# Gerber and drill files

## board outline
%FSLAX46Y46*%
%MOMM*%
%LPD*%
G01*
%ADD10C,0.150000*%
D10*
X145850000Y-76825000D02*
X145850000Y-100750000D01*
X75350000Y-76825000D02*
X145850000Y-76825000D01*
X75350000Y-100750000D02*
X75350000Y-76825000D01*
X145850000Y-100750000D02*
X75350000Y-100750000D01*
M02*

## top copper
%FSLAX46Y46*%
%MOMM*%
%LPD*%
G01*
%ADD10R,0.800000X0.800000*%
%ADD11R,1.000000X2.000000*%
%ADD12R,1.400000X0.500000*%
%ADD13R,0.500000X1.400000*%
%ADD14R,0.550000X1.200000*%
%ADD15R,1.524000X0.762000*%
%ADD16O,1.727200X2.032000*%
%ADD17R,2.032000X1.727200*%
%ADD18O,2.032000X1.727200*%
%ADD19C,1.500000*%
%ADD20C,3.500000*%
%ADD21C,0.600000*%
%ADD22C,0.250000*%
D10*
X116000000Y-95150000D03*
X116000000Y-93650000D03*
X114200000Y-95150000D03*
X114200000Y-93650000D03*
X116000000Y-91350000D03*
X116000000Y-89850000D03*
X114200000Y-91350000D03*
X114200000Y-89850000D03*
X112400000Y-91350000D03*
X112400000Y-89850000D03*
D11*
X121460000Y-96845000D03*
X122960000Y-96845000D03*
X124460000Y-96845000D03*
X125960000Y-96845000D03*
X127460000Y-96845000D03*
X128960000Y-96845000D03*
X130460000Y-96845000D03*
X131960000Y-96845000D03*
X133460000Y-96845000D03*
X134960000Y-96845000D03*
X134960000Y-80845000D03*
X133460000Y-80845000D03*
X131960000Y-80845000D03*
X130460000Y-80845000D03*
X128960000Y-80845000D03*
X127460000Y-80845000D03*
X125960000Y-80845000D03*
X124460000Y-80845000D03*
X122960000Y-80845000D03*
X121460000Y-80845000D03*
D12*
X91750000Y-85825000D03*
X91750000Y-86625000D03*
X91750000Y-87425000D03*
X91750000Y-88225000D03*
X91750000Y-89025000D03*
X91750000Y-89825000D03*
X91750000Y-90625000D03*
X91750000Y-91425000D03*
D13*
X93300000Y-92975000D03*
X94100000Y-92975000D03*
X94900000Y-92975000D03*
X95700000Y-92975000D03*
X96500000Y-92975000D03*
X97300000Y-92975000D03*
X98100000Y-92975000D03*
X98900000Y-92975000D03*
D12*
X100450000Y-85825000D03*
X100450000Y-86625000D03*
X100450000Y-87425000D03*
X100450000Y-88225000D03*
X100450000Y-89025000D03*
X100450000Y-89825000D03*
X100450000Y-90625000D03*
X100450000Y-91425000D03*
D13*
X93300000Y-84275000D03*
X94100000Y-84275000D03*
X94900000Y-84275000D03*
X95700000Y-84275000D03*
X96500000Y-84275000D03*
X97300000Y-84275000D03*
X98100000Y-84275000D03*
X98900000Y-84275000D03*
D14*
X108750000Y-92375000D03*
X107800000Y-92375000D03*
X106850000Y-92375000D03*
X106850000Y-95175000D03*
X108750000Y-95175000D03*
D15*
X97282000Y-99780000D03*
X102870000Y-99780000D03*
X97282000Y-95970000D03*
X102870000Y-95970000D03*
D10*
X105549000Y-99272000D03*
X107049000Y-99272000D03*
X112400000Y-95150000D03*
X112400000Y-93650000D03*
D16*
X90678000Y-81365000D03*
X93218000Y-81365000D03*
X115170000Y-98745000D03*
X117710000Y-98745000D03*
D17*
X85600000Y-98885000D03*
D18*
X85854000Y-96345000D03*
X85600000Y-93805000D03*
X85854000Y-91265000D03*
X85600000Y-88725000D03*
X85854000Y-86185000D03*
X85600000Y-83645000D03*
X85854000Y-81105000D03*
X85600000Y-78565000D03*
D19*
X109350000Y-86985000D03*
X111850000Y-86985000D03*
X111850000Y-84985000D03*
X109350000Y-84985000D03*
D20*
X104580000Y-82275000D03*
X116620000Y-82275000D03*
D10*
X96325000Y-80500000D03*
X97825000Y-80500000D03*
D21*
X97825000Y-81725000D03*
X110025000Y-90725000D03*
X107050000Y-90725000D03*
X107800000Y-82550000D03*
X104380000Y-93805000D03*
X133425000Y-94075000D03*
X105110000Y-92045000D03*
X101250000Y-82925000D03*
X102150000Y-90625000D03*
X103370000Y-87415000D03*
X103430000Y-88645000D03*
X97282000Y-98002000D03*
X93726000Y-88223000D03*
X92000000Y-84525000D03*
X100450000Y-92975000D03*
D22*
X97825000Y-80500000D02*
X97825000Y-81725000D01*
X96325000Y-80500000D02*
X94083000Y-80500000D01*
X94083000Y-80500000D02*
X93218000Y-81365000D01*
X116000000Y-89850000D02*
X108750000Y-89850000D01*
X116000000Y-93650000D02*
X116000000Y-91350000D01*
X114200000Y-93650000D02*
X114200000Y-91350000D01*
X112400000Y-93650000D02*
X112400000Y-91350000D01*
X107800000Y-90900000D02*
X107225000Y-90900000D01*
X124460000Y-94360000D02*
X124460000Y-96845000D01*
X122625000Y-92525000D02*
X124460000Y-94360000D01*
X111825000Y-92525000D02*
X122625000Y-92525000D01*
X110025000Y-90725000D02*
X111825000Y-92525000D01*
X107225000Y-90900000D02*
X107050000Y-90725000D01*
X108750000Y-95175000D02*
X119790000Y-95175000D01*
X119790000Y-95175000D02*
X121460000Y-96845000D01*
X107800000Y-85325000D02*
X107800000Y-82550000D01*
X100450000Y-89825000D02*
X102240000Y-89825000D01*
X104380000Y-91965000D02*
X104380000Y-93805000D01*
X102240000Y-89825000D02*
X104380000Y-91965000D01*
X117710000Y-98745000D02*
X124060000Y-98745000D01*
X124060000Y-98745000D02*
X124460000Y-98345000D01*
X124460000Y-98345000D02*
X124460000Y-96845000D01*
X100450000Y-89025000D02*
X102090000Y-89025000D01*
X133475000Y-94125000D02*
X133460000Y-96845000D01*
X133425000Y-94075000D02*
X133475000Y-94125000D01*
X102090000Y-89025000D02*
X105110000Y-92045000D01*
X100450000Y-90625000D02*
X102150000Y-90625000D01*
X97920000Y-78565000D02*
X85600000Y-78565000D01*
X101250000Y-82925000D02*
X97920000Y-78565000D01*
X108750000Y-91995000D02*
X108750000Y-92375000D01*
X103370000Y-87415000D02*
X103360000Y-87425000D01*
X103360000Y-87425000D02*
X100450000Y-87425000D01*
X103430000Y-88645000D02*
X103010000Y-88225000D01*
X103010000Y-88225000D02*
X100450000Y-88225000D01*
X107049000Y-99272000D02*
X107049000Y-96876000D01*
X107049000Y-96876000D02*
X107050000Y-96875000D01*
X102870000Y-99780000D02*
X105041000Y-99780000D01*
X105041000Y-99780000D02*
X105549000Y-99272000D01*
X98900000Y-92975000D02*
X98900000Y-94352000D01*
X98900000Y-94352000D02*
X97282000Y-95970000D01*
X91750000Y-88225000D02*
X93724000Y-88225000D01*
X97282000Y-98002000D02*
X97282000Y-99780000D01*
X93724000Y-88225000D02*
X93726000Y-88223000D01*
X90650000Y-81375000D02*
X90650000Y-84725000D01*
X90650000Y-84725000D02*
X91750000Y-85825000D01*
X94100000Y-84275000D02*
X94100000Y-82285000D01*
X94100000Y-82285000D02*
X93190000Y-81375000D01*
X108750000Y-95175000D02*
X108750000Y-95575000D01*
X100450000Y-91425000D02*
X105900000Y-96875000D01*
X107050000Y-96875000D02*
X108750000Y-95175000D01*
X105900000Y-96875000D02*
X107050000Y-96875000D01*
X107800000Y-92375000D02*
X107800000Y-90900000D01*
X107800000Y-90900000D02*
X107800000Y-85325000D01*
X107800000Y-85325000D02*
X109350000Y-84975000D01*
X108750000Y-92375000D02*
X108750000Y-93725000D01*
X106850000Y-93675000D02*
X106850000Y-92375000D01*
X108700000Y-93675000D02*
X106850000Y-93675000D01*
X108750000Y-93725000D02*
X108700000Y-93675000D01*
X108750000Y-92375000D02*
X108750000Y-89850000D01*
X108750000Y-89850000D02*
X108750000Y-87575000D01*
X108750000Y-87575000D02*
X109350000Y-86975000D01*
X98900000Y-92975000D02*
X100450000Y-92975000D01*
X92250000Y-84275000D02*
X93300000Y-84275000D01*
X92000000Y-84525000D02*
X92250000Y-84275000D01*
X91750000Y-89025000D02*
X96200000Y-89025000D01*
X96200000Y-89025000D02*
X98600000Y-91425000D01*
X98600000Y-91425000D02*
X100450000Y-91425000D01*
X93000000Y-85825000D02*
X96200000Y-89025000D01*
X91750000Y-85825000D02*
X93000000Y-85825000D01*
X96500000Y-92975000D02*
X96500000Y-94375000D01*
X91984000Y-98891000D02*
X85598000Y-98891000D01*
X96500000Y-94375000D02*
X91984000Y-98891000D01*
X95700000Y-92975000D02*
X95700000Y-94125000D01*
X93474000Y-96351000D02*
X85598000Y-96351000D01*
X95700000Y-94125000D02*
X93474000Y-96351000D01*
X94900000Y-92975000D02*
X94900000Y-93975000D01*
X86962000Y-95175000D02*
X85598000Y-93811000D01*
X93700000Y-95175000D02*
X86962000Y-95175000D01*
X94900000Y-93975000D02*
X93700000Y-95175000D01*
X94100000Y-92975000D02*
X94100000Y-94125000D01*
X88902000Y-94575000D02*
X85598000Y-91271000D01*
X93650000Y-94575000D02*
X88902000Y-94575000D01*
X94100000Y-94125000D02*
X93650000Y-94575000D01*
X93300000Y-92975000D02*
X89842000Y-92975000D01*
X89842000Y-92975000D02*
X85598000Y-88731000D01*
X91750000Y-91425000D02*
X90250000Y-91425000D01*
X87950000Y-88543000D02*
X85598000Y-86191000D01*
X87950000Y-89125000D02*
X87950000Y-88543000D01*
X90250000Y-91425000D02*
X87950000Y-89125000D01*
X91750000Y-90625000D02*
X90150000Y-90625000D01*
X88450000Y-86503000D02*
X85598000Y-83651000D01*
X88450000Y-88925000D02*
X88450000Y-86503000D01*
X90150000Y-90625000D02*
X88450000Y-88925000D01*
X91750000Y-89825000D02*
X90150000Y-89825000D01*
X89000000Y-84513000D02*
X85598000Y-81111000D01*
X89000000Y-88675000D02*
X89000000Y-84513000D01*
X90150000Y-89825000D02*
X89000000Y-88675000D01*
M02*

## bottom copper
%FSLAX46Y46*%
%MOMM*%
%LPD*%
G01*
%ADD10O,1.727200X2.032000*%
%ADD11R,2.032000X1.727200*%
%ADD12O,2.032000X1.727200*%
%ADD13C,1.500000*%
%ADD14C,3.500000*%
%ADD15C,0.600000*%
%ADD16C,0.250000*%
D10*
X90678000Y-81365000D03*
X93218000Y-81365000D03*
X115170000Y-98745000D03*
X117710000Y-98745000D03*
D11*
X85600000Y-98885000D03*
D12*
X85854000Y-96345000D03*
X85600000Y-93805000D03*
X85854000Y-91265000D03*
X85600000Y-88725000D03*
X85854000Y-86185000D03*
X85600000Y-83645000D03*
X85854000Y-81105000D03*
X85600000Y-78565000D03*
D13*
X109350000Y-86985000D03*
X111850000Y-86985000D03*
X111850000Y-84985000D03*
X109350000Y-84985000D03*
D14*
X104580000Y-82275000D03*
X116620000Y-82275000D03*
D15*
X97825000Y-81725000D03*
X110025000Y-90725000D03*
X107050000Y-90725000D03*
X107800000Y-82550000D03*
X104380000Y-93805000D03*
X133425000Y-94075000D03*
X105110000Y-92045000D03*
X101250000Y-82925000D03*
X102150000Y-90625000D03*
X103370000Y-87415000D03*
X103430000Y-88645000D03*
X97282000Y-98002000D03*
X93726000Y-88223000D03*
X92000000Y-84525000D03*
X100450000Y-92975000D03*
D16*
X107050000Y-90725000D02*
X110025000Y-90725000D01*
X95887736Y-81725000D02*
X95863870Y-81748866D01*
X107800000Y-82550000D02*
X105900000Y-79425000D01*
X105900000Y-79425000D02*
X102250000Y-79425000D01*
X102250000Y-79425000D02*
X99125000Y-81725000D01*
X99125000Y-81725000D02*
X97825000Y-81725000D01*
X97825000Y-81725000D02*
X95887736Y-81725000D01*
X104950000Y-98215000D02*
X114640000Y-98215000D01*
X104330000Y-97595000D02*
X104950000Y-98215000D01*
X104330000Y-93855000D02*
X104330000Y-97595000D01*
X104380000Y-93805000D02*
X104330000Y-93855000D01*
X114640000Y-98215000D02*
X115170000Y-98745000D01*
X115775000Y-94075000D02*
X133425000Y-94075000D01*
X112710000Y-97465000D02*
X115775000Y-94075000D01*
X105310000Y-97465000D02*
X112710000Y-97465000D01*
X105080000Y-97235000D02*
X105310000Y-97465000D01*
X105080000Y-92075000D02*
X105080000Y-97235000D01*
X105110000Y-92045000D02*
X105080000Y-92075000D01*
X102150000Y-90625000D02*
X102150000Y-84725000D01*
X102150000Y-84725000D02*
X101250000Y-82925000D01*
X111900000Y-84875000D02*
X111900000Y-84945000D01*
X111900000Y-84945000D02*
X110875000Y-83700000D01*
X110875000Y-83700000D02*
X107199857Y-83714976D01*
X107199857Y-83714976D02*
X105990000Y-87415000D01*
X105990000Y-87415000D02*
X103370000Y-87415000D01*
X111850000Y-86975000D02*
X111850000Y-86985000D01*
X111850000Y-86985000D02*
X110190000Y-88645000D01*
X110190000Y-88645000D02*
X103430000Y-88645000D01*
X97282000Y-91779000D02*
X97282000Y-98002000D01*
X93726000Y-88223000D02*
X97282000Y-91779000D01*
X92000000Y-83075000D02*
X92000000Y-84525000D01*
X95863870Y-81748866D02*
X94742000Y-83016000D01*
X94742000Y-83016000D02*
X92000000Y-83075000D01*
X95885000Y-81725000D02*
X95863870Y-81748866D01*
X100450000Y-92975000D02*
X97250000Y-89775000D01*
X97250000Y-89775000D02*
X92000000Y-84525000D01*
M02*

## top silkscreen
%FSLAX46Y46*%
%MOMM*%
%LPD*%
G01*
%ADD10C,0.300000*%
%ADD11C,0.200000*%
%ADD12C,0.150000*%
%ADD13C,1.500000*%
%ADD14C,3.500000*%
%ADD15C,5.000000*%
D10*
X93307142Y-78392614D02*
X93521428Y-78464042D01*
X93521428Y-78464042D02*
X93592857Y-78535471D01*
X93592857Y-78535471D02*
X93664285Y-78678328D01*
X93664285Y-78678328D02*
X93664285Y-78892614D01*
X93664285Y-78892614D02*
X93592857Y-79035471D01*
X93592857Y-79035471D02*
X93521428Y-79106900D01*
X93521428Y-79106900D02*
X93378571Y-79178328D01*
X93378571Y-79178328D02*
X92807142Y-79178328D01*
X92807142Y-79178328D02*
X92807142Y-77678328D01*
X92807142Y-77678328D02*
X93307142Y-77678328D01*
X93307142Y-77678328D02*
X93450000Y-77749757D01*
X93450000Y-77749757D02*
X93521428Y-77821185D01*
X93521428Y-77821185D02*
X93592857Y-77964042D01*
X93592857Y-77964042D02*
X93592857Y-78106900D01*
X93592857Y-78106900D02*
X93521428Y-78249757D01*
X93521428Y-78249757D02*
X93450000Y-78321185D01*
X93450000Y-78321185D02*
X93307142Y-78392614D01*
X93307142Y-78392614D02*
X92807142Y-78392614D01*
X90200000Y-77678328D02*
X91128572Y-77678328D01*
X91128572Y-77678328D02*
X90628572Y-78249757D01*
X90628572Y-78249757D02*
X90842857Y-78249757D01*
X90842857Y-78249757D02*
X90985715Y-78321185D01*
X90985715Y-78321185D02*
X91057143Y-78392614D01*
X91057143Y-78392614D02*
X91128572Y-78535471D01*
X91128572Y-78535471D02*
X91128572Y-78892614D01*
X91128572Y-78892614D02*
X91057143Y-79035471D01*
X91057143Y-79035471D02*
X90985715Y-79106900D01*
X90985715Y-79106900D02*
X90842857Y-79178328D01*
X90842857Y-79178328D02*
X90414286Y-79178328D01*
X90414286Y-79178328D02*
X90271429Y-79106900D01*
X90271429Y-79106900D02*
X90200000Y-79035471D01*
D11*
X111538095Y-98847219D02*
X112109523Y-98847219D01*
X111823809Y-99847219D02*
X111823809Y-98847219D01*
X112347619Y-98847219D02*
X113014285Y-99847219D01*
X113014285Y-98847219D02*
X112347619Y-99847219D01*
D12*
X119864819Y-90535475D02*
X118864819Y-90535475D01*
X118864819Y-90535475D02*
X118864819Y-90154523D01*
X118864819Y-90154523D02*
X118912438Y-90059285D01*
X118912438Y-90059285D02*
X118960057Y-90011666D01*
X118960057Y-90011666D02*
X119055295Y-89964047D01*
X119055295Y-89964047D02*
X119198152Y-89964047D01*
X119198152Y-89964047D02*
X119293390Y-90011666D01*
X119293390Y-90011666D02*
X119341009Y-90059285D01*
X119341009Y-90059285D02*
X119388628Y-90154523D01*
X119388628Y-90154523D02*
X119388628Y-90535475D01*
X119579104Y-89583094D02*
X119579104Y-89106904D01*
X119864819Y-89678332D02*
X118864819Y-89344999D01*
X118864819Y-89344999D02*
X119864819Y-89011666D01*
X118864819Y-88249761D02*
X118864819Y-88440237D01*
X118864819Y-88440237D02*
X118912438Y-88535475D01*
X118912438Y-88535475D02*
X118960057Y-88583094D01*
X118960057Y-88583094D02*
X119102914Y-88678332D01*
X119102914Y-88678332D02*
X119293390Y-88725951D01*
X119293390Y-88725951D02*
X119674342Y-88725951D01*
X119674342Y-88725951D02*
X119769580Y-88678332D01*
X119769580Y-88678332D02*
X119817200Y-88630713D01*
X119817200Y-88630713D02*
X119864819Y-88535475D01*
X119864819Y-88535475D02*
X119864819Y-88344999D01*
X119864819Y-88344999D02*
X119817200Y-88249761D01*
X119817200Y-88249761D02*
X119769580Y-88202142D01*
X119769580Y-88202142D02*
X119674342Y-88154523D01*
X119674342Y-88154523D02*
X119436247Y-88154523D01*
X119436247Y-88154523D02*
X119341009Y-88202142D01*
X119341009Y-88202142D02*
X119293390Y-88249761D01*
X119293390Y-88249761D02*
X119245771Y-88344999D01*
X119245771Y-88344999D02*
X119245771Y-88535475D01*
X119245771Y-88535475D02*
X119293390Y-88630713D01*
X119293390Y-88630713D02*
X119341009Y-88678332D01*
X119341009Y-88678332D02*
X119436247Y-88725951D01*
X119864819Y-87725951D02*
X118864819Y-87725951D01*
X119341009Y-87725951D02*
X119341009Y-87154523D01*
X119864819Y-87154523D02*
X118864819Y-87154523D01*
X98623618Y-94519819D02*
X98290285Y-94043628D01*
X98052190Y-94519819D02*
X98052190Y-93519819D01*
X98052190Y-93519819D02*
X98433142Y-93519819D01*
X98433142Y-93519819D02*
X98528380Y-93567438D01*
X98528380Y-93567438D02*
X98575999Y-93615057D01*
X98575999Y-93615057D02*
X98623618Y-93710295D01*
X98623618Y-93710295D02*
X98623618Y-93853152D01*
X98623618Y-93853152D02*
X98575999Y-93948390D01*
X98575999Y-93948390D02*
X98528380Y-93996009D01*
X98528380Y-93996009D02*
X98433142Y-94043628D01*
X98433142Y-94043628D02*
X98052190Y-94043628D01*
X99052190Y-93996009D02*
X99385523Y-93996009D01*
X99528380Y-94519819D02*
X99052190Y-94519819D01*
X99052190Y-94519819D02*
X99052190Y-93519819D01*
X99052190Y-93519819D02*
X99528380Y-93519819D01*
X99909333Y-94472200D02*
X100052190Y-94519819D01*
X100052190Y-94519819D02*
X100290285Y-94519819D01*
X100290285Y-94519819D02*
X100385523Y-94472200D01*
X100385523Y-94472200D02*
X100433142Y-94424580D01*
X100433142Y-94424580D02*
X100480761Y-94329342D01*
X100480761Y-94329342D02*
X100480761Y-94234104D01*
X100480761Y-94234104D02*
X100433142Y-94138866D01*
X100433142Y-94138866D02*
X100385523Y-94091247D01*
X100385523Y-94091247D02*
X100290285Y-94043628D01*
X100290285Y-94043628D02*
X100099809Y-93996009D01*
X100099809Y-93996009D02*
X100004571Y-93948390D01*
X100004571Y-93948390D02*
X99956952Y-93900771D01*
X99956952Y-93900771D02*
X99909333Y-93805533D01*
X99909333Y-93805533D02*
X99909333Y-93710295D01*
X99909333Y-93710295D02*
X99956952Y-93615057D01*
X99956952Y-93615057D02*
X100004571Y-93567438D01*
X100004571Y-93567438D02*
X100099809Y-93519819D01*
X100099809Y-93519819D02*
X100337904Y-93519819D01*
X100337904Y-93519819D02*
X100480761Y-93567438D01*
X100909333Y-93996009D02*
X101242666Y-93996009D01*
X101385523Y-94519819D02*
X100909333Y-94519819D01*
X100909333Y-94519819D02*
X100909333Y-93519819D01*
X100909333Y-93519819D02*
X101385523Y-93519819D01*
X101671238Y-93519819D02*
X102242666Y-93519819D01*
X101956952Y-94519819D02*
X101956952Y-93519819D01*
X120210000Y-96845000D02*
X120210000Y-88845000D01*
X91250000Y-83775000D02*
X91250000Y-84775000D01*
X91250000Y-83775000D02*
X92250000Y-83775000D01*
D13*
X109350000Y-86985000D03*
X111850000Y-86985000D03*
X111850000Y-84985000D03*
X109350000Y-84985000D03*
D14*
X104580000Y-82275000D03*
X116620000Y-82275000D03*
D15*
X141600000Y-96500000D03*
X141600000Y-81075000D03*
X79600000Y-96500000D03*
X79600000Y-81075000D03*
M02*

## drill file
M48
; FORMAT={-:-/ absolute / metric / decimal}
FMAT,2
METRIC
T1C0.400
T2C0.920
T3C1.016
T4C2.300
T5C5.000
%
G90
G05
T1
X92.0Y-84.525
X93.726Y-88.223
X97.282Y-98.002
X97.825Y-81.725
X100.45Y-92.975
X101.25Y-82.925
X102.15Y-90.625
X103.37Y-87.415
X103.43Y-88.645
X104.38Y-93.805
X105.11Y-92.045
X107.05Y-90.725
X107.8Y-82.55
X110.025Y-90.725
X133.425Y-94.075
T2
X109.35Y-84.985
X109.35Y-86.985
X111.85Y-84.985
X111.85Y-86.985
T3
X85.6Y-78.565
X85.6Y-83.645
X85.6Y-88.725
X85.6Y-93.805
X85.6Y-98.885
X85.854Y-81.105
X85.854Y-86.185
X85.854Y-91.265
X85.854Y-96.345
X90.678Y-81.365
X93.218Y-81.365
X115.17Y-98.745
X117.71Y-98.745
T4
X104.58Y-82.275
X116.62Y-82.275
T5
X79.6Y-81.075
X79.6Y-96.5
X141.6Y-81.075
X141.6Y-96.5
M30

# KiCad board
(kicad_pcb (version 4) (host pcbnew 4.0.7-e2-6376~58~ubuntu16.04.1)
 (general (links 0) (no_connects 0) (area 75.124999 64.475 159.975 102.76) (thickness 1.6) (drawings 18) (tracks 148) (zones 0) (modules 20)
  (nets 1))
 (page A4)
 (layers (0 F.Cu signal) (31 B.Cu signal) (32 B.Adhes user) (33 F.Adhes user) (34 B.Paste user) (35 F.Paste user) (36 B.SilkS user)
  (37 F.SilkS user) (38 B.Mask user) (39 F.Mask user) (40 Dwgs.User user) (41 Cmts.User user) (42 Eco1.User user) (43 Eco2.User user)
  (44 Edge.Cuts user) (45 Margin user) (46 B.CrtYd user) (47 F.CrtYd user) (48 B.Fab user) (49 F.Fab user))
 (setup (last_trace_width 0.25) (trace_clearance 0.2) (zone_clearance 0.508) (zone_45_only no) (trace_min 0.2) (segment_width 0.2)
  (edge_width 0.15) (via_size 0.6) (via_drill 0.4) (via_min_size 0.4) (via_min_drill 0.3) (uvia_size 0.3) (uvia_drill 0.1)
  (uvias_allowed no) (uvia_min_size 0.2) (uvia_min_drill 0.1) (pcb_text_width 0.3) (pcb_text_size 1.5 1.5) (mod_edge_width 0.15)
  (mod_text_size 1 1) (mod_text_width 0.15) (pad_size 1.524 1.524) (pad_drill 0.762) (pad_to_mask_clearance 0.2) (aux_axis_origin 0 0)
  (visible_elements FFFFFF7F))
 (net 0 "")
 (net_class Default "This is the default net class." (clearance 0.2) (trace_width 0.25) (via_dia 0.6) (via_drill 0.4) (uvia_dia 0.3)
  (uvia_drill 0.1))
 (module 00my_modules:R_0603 (layer F.Cu) (at 116 94.4 90)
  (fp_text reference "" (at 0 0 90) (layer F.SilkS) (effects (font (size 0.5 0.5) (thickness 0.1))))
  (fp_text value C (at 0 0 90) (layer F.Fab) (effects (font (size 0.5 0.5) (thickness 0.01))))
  (pad 1 smd rect (at -0.75 0 90) (size 0.8 0.8) (layers F.Cu F.Paste F.Mask))
  (pad 2 smd rect (at 0.75 0 90) (size 0.8 0.8) (layers F.Cu F.Paste F.Mask)))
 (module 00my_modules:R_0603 (layer F.Cu) (at 114.2 94.4 90)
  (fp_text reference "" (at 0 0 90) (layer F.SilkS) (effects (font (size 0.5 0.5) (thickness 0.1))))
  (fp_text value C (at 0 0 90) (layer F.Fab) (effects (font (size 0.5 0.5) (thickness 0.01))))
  (pad 1 smd rect (at -0.75 0 90) (size 0.8 0.8) (layers F.Cu F.Paste F.Mask))
  (pad 2 smd rect (at 0.75 0 90) (size 0.8 0.8) (layers F.Cu F.Paste F.Mask)))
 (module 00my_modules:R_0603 (layer F.Cu) (at 116 90.6 90)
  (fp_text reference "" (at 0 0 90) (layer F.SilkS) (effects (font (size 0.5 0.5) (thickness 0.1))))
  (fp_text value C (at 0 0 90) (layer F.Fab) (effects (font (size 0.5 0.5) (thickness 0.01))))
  (pad 1 smd rect (at -0.75 0 90) (size 0.8 0.8) (layers F.Cu F.Paste F.Mask))
  (pad 2 smd rect (at 0.75 0 90) (size 0.8 0.8) (layers F.Cu F.Paste F.Mask)))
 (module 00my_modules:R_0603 (layer F.Cu) (at 114.2 90.6 90)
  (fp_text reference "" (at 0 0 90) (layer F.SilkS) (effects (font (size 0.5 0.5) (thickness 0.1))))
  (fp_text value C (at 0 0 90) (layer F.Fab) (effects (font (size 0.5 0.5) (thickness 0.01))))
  (pad 1 smd rect (at -0.75 0 90) (size 0.8 0.8) (layers F.Cu F.Paste F.Mask))
  (pad 2 smd rect (at 0.75 0 90) (size 0.8 0.8) (layers F.Cu F.Paste F.Mask)))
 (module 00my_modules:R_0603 (layer F.Cu) (at 112.4 90.6 90)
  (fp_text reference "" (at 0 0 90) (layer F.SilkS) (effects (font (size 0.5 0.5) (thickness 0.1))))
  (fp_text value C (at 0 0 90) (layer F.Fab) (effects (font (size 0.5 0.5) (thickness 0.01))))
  (pad 1 smd rect (at -0.75 0 90) (size 0.8 0.8) (layers F.Cu F.Paste F.Mask))
  (pad 2 smd rect (at 0.75 0 90) (size 0.8 0.8) (layers F.Cu F.Paste F.Mask)))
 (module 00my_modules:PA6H (layer F.Cu) (at 128.21 88.845 90)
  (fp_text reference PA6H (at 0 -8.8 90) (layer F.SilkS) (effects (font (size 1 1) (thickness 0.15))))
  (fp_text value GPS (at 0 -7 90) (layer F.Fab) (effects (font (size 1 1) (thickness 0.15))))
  (fp_line (start -8 -8) (end 0 -8) (layer F.SilkS) (width 0.15))
  (pad VCC smd rect (at -8 -6.75 90) (size 2 1) (layers F.Cu F.Paste F.Mask))
  (pad 2 smd rect (at -8 -5.25 90) (size 2 1) (layers F.Cu F.Paste F.Mask))
  (pad GND smd rect (at -8 -3.75 90) (size 2 1) (layers F.Cu F.Paste F.Mask))
  (pad 4 smd rect (at -8 -2.25 90) (size 2 1) (layers F.Cu F.Paste F.Mask))
  (pad 5 smd rect (at -8 -0.75 90) (size 2 1) (layers F.Cu F.Paste F.Mask))
  (pad 6 smd rect (at -8 0.75 90) (size 2 1) (layers F.Cu F.Paste F.Mask))
  (pad 7 smd rect (at -8 2.25 90) (size 2 1) (layers F.Cu F.Paste F.Mask))
  (pad 8 smd rect (at -8 3.75 90) (size 2 1) (layers F.Cu F.Paste F.Mask))
  (pad TX smd rect (at -8 5.25 90) (size 2 1) (layers F.Cu F.Paste F.Mask))
  (pad RX smd rect (at -8 6.75 90) (size 2 1) (layers F.Cu F.Paste F.Mask))
  (pad 11 smd rect (at 8 6.75 90) (size 2 1) (layers F.Cu F.Paste F.Mask))
  (pad 12 smd rect (at 8 5.25 90) (size 2 1) (layers F.Cu F.Paste F.Mask))
  (pad 13 smd rect (at 8 3.75 90) (size 2 1) (layers F.Cu F.Paste F.Mask))
  (pad 14 smd rect (at 8 2.25 90) (size 2 1) (layers F.Cu F.Paste F.Mask))
  (pad 15 smd rect (at 8 0.75 90) (size 2 1) (layers F.Cu F.Paste F.Mask))
  (pad 16 smd rect (at 8 -0.75 90) (size 2 1) (layers F.Cu F.Paste F.Mask))
  (pad 17 smd rect (at 8 -2.25 90) (size 2 1) (layers F.Cu F.Paste F.Mask))
  (pad 18 smd rect (at 8 -3.75 90) (size 2 1) (layers F.Cu F.Paste F.Mask))
  (pad 19 smd rect (at 8 -5.25 90) (size 2 1) (layers F.Cu F.Paste F.Mask))
  (pad 20 smd rect (at 8 -6.75 90) (size 2 1) (layers F.Cu F.Paste F.Mask)))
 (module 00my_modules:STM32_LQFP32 (layer F.Cu) (at 96.1 88.625)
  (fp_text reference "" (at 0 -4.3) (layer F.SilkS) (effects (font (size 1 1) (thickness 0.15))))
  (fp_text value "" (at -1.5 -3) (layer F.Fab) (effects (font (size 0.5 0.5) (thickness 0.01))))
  (fp_line (start -4.85 -4.85) (end -4.85 -3.85) (layer F.SilkS) (width 0.15))
  (fp_line (start -4.85 -4.85) (end -3.85 -4.85) (layer F.SilkS) (width 0.15))
  (pad 3.3 smd rect (at -4.35 -2.8) (size 1.4 0.5) (layers F.Cu F.Paste F.Mask))
  (pad PF0 smd rect (at -4.35 -2) (size 1.4 0.5) (layers F.Cu F.Paste F.Mask))
  (pad PF1 smd rect (at -4.35 -1.2) (size 1.4 0.5) (layers F.Cu F.Paste F.Mask))
  (pad RST smd rect (at -4.35 -0.4) (size 1.4 0.5) (layers F.Cu F.Paste F.Mask))
  (pad 3.3 smd rect (at -4.35 0.4) (size 1.4 0.5) (layers F.Cu F.Paste F.Mask))
  (pad PA0 smd rect (at -4.35 1.2) (size 1.4 0.5) (layers F.Cu F.Paste F.Mask))
  (pad PA1 smd rect (at -4.35 2) (size 1.4 0.5) (layers F.Cu F.Paste F.Mask))
  (pad PA2 smd rect (at -4.35 2.8) (size 1.4 0.5) (layers F.Cu F.Paste F.Mask))
  (pad PA3 smd rect (at -2.8 4.35 90) (size 1.4 0.5) (layers F.Cu F.Paste F.Mask))
  (pad PA4 smd rect (at -2 4.35 90) (size 1.4 0.5) (layers F.Cu F.Paste F.Mask))
  (pad PA5 smd rect (at -1.2 4.35 90) (size 1.4 0.5) (layers F.Cu F.Paste F.Mask))
  (pad PA6 smd rect (at -0.4 4.35 90) (size 1.4 0.5) (layers F.Cu F.Paste F.Mask))
  (pad PA7 smd rect (at 0.4 4.35 90) (size 1.4 0.5) (layers F.Cu F.Paste F.Mask))
  (pad PB0 smd rect (at 1.2 4.35 90) (size 1.4 0.5) (layers F.Cu F.Paste F.Mask))
  (pad PB1 smd rect (at 2 4.35 90) (size 1.4 0.5) (layers F.Cu F.Paste F.Mask))
  (pad GND smd rect (at 2.8 4.35 90) (size 1.4 0.5) (layers F.Cu F.Paste F.Mask))
  (pad PA14 smd rect (at 4.35 -2.8) (size 1.4 0.5) (layers F.Cu F.Paste F.Mask))
  (pad PA13 smd rect (at 4.35 -2) (size 1.4 0.5) (layers F.Cu F.Paste F.Mask))
  (pad PA12 smd rect (at 4.35 -1.2) (size 1.4 0.5) (layers F.Cu F.Paste F.Mask))
  (pad PA11 smd rect (at 4.35 -0.4) (size 1.4 0.5) (layers F.Cu F.Paste F.Mask))
  (pad PA10 smd rect (at 4.35 0.4) (size 1.4 0.5) (layers F.Cu F.Paste F.Mask))
  (pad PA9 smd rect (at 4.35 1.2) (size 1.4 0.5) (layers F.Cu F.Paste F.Mask))
  (pad PA8 smd rect (at 4.35 2) (size 1.4 0.5) (layers F.Cu F.Paste F.Mask))
  (pad 3.3 smd rect (at 4.35 2.8) (size 1.4 0.5) (layers F.Cu F.Paste F.Mask))
  (pad GND smd rect (at -2.8 -4.35 90) (size 1.4 0.5) (layers F.Cu F.Paste F.Mask))
  (pad BOOT smd rect (at -2 -4.35 90) (size 1.4 0.5) (layers F.Cu F.Paste F.Mask))
  (pad PB7 smd rect (at -1.2 -4.35 90) (size 1.4 0.5) (layers F.Cu F.Paste F.Mask))
  (pad PB6 smd rect (at -0.4 -4.35 90) (size 1.4 0.5) (layers F.Cu F.Paste F.Mask))
  (pad PB5 smd rect (at 0.4 -4.35 90) (size 1.4 0.5) (layers F.Cu F.Paste F.Mask))
  (pad PB4 smd rect (at 1.2 -4.35 90) (size 1.4 0.5) (layers F.Cu F.Paste F.Mask))
  (pad PB3 smd rect (at 2 -4.35 90) (size 1.4 0.5) (layers F.Cu F.Paste F.Mask))
  (pad PA15 smd rect (at 2.8 -4.35 90) (size 1.4 0.5) (layers F.Cu F.Paste F.Mask)))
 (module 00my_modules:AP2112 (layer F.Cu) (at 107.8 93.775 270)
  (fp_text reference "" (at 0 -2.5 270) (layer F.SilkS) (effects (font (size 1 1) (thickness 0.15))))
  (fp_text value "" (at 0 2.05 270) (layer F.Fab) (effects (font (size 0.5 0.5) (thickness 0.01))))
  (pad VIN smd rect (at -1.4 -0.95 270) (size 1.2 0.55) (layers F.Cu F.Paste F.Mask))
  (pad GND smd rect (at -1.4 0 270) (size 1.2 0.55) (layers F.Cu F.Paste F.Mask))
  (pad EN smd rect (at -1.4 0.95 270) (size 1.2 0.55) (layers F.Cu F.Paste F.Mask))
  (pad NC smd rect (at 1.4 0.95 270) (size 1.2 0.55) (layers F.Cu F.Paste F.Mask))
  (pad VOUT smd rect (at 1.4 -0.95 270) (size 1.2 0.55) (layers F.Cu F.Paste F.Mask)))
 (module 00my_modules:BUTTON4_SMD (layer F.Cu) (at 100.076 97.875)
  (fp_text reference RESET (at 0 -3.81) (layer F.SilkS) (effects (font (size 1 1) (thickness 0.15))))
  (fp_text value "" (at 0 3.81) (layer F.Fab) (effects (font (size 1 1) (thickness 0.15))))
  (pad 1 smd rect (at -2.794 1.905) (size 1.524 0.762) (layers F.Cu F.Paste F.Mask))
  (pad 2 smd rect (at 2.794 1.905) (size 1.524 0.762) (layers F.Cu F.Paste F.Mask))
  (pad 3 smd rect (at -2.794 -1.905) (size 1.524 0.762) (layers F.Cu F.Paste F.Mask))
  (pad 4 smd rect (at 2.794 -1.905) (size 1.524 0.762) (layers F.Cu F.Paste F.Mask)))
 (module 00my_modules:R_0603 (layer F.Cu) (at 106.299 99.272)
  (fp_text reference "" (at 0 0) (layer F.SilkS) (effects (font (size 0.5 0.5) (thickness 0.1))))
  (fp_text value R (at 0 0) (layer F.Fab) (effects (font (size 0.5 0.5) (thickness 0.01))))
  (pad 1 smd rect (at -0.75 0) (size 0.8 0.8) (layers F.Cu F.Paste F.Mask))
  (pad 2 smd rect (at 0.75 0) (size 0.8 0.8) (layers F.Cu F.Paste F.Mask)))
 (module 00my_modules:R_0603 (layer F.Cu) (at 112.4 94.4 90)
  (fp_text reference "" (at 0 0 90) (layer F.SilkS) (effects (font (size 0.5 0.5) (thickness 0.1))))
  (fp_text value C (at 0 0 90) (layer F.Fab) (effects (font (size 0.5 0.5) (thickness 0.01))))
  (pad 1 smd rect (at -0.75 0 90) (size 0.8 0.8) (layers F.Cu F.Paste F.Mask))
  (pad 2 smd rect (at 0.75 0 90) (size 0.8 0.8) (layers F.Cu F.Paste F.Mask)))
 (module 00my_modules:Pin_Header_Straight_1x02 (layer B.Cu) (at 90.678 81.365 270)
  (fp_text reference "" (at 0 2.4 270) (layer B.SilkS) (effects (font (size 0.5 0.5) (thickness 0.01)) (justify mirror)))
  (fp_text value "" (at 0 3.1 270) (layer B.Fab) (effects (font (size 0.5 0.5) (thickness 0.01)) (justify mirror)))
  (pad 1 thru_hole oval (at 0 0 270) (size 2.032 1.7272) (drill 1.016) (layers *.Cu *.Mask B.SilkS))
  (pad 2 thru_hole oval (at 0 -2.54 270) (size 2.032 1.7272) (drill 1.016) (layers *.Cu *.Mask B.SilkS)))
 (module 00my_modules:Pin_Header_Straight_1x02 (layer B.Cu) (at 115.17 98.745 270)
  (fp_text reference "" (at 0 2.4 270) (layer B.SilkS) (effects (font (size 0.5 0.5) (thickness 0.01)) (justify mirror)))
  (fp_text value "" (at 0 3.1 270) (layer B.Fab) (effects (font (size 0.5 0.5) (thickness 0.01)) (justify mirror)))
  (pad 1 thru_hole oval (at 0 0 270) (size 2.032 1.7272) (drill 1.016) (layers *.Cu *.Mask B.SilkS))
  (pad 2 thru_hole oval (at 0 -2.54 270) (size 2.032 1.7272) (drill 1.016) (layers *.Cu *.Mask B.SilkS)))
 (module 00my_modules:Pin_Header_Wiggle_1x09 (layer B.Cu) (at 85.6 98.885)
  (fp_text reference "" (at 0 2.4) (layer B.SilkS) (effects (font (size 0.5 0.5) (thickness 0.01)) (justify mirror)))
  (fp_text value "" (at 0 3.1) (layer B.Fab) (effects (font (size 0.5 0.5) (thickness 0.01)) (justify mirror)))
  (pad 1 thru_hole rect (at 0 0) (size 2.032 1.7272) (drill 1.016) (layers *.Cu *.Mask B.SilkS))
  (pad 2 thru_hole oval (at 0.254 -2.54) (size 2.032 1.7272) (drill 1.016) (layers *.Cu *.Mask B.SilkS))
  (pad 3 thru_hole oval (at 0 -5.08) (size 2.032 1.7272) (drill 1.016) (layers *.Cu *.Mask B.SilkS))
  (pad 4 thru_hole oval (at 0.254 -7.62) (size 2.032 1.7272) (drill 1.016) (layers *.Cu *.Mask B.SilkS))
  (pad 5 thru_hole oval (at 0 -10.16) (size 2.032 1.7272) (drill 1.016) (layers *.Cu *.Mask B.SilkS))
  (pad 6 thru_hole oval (at 0.254 -12.7) (size 2.032 1.7272) (drill 1.016) (layers *.Cu *.Mask B.SilkS))
  (pad 7 thru_hole oval (at 0 -15.24) (size 2.032 1.7272) (drill 1.016) (layers *.Cu *.Mask B.SilkS))
  (pad 8 thru_hole oval (at 0.254 -17.78) (size 2.032 1.7272) (drill 1.016) (layers *.Cu *.Mask B.SilkS))
  (pad 9 thru_hole oval (at 0 -20.32) (size 2.032 1.7272) (drill 1.016) (layers *.Cu *.Mask B.SilkS)))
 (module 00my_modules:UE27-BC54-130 (layer F.Cu) (at 110.6 82.275 180)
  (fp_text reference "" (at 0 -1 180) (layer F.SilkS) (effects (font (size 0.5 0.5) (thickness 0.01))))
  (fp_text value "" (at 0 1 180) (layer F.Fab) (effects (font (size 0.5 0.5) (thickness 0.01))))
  (pad V thru_hole circle (at 1.25 -4.71 180) (size 1.5 1.5) (drill 0.92) (layers *.Cu *.Mask F.SilkS))
  (pad - thru_hole circle (at -1.25 -4.71 180) (size 1.5 1.5) (drill 0.92) (layers *.Cu *.Mask F.SilkS))
  (pad + thru_hole circle (at -1.25 -2.71 180) (size 1.5 1.5) (drill 0.92) (layers *.Cu *.Mask F.SilkS))
  (pad G thru_hole circle (at 1.25 -2.71 180) (size 1.5 1.5) (drill 0.92) (layers *.Cu *.Mask F.SilkS))
  (pad X thru_hole circle (at 6.02 0 180) (size 3.5 3.5) (drill 2.3) (layers *.Cu *.Mask F.SilkS))
  (pad X thru_hole circle (at -6.02 0 180) (size 3.5 3.5) (drill 2.3) (layers *.Cu *.Mask F.SilkS)))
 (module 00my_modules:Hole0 (layer F.Cu) (at 141.6 96.5)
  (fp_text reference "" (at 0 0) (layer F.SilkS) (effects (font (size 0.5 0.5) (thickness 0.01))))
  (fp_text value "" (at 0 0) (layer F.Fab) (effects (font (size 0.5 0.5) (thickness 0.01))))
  (pad "" np_thru_hole circle (at 0 0) (size 5 5) (drill 5) (layers *.Cu *.Mask F.SilkS)))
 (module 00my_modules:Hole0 (layer F.Cu) (at 141.6 81.075)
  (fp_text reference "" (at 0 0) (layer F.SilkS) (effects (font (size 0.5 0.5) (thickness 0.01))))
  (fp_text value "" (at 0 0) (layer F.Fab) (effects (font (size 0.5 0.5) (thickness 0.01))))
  (pad "" np_thru_hole circle (at 0 0) (size 5 5) (drill 5) (layers *.Cu *.Mask F.SilkS)))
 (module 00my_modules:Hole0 (layer F.Cu) (at 79.6 96.5)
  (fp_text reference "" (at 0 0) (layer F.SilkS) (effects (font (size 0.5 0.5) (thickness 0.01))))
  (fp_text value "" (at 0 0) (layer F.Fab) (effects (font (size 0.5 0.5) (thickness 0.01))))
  (pad "" np_thru_hole circle (at 0 0) (size 5 5) (drill 5) (layers *.Cu *.Mask F.SilkS)))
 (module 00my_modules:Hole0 (layer F.Cu) (at 79.6 81.075)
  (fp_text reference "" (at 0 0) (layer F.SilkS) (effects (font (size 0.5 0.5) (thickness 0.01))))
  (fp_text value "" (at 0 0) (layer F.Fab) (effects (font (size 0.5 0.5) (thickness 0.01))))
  (pad "" np_thru_hole circle (at 0 0) (size 5 5) (drill 5) (layers *.Cu *.Mask F.SilkS)))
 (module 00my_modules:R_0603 (layer F.Cu) (at 97.075 80.5)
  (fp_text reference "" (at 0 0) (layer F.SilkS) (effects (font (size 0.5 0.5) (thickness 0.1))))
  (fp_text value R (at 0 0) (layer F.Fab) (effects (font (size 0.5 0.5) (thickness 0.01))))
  (pad 1 smd rect (at -0.75 0) (size 0.8 0.8) (layers F.Cu F.Paste F.Mask))
  (pad 2 smd rect (at 0.75 0) (size 0.8 0.8) (layers F.Cu F.Paste F.Mask)))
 (gr_line (start 145.85 76.825) (end 145.85 100.75) (angle 90) (layer Edge.Cuts) (width 0.15))
 (gr_line (start 75.35 76.825) (end 145.85 76.825) (angle 90) (layer Edge.Cuts) (width 0.15))
 (gr_line (start 75.35 100.75) (end 75.35 76.825) (angle 90) (layer Edge.Cuts) (width 0.15))
 (gr_line (start 145.85 100.75) (end 75.35 100.75) (angle 90) (layer Edge.Cuts) (width 0.15))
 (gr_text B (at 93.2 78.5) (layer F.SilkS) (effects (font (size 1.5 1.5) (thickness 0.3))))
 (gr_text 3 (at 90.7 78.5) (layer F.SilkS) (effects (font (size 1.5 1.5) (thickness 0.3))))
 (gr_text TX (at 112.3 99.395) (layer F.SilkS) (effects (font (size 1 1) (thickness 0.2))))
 (segment (start 97.825 80.5) (end 97.825 81.725) (width 0.25) (layer F.Cu) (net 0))
 (via (at 97.825 81.725) (size 0.6) (drill 0.4) (layers F.Cu B.Cu) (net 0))
 (segment (start 96.325 80.5) (end 94.083 80.5) (width 0.25) (layer F.Cu) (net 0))
 (segment (start 94.083 80.5) (end 93.218 81.365) (width 0.25) (layer F.Cu) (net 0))
 (segment (start 116 89.85) (end 108.75 89.85) (width 0.25) (layer F.Cu) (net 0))
 (segment (start 116 93.65) (end 116 91.35) (width 0.25) (layer F.Cu) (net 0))
 (segment (start 114.2 93.65) (end 114.2 91.35) (width 0.25) (layer F.Cu) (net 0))
 (segment (start 112.4 93.65) (end 112.4 91.35) (width 0.25) (layer F.Cu) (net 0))
 (segment (start 107.8 90.9) (end 107.225 90.9) (width 0.25) (layer F.Cu) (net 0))
 (segment (start 124.46 94.36) (end 124.46 96.845) (width 0.25) (layer F.Cu) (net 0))
 (segment (start 122.625 92.525) (end 124.46 94.36) (width 0.25) (layer F.Cu) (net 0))
 (segment (start 111.825 92.525) (end 122.625 92.525) (width 0.25) (layer F.Cu) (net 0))
 (segment (start 110.025 90.725) (end 111.825 92.525) (width 0.25) (layer F.Cu) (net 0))
 (via (at 110.025 90.725) (size 0.6) (drill 0.4) (layers F.Cu B.Cu) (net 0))
 (segment (start 107.05 90.725) (end 110.025 90.725) (width 0.25) (layer B.Cu) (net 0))
 (via (at 107.05 90.725) (size 0.6) (drill 0.4) (layers F.Cu B.Cu) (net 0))
 (segment (start 107.225 90.9) (end 107.05 90.725) (width 0.25) (layer F.Cu) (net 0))
 (segment (start 108.75 95.175) (end 119.79 95.175) (width 0.25) (layer F.Cu) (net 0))
 (segment (start 119.79 95.175) (end 121.46 96.845) (width 0.25) (layer F.Cu) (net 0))
 (segment (start 107.8 85.325) (end 107.8 82.55) (width 0.25) (layer F.Cu) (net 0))
 (segment (start 95.887736 81.725) (end 95.86387 81.748866) (width 0.25) (layer B.Cu) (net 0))
 (segment (start 107.8 82.55) (end 105.9 79.425) (width 0.25) (layer B.Cu) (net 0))
 (segment (start 105.9 79.425) (end 102.25 79.425) (width 0.25) (layer B.Cu) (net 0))
 (segment (start 102.25 79.425) (end 99.125 81.725) (width 0.25) (layer B.Cu) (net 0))
 (segment (start 99.125 81.725) (end 97.825 81.725) (width 0.25) (layer B.Cu) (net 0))
 (segment (start 97.825 81.725) (end 95.887736 81.725) (width 0.25) (layer B.Cu) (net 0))
 (via (at 107.8 82.55) (size 0.6) (drill 0.4) (layers F.Cu B.Cu) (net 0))
 (segment (start 100.45 89.825) (end 102.24 89.825) (width 0.25) (layer F.Cu) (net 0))
 (segment (start 104.95 98.215) (end 114.64 98.215) (width 0.25) (layer B.Cu) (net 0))
 (segment (start 104.33 97.595) (end 104.95 98.215) (width 0.25) (layer B.Cu) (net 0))
 (segment (start 104.33 93.855) (end 104.33 97.595) (width 0.25) (layer B.Cu) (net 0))
 (segment (start 104.38 93.805) (end 104.33 93.855) (width 0.25) (layer B.Cu) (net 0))
 (via (at 104.38 93.805) (size 0.6) (drill 0.4) (layers F.Cu B.Cu) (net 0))
 (segment (start 104.38 91.965) (end 104.38 93.805) (width 0.25) (layer F.Cu) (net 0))
 (segment (start 102.24 89.825) (end 104.38 91.965) (width 0.25) (layer F.Cu) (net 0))
 (segment (start 114.64 98.215) (end 115.17 98.745) (width 0.25) (layer B.Cu) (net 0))
 (segment (start 117.71 98.745) (end 124.06 98.745) (width 0.25) (layer F.Cu) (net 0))
 (segment (start 124.06 98.745) (end 124.46 98.345) (width 0.25) (layer F.Cu) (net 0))
 (segment (start 124.46 98.345) (end 124.46 96.845) (width 0.25) (layer F.Cu) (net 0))
 (segment (start 100.45 89.025) (end 102.09 89.025) (width 0.25) (layer F.Cu) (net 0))
 (segment (start 133.475 94.125) (end 133.46 96.845) (width 0.25) (layer F.Cu) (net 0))
 (segment (start 133.425 94.075) (end 133.475 94.125) (width 0.25) (layer F.Cu) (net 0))
 (via (at 133.425 94.075) (size 0.6) (drill 0.4) (layers F.Cu B.Cu) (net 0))
 (segment (start 115.775 94.075) (end 133.425 94.075) (width 0.25) (layer B.Cu) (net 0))
 (segment (start 112.71 97.465) (end 115.775 94.075) (width 0.25) (layer B.Cu) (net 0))
 (segment (start 105.31 97.465) (end 112.71 97.465) (width 0.25) (layer B.Cu) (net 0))
 (segment (start 105.08 97.235) (end 105.31 97.465) (width 0.25) (layer B.Cu) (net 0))
 (segment (start 105.08 92.075) (end 105.08 97.235) (width 0.25) (layer B.Cu) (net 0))
 (segment (start 105.11 92.045) (end 105.08 92.075) (width 0.25) (layer B.Cu) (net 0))
 (via (at 105.11 92.045) (size 0.6) (drill 0.4) (layers F.Cu B.Cu) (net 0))
 (segment (start 102.09 89.025) (end 105.11 92.045) (width 0.25) (layer F.Cu) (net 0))
 (segment (start 100.45 90.625) (end 102.15 90.625) (width 0.25) (layer F.Cu) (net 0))
 (segment (start 97.92 78.565) (end 85.6 78.565) (width 0.25) (layer F.Cu) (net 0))
 (segment (start 101.25 82.925) (end 97.92 78.565) (width 0.25) (layer F.Cu) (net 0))
 (via (at 101.25 82.925) (size 0.6) (drill 0.4) (layers F.Cu B.Cu) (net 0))
 (segment (start 102.15 90.625) (end 102.15 84.725) (width 0.25) (layer B.Cu) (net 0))
 (segment (start 102.15 84.725) (end 101.25 82.925) (width 0.25) (layer B.Cu) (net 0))
 (via (at 102.15 90.625) (size 0.6) (drill 0.4) (layers F.Cu B.Cu) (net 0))
 (segment (start 108.75 91.995) (end 108.75 92.375) (width 0.25) (layer F.Cu) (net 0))
 (segment (start 111.9 84.875) (end 111.9 84.945) (width 0.25) (layer B.Cu) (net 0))
 (segment (start 111.9 84.945) (end 110.875 83.7) (width 0.25) (layer B.Cu) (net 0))
 (segment (start 110.875 83.7) (end 107.199857 83.714976) (width 0.25) (layer B.Cu) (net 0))
 (segment (start 107.199857 83.714976) (end 105.99 87.415) (width 0.25) (layer B.Cu) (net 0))
 (segment (start 105.99 87.415) (end 103.37 87.415) (width 0.25) (layer B.Cu) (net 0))
 (via (at 103.37 87.415) (size 0.6) (drill 0.4) (layers F.Cu B.Cu) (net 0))
 (segment (start 103.37 87.415) (end 103.36 87.425) (width 0.25) (layer F.Cu) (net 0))
 (segment (start 103.36 87.425) (end 100.45 87.425) (width 0.25) (layer F.Cu) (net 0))
 (segment (start 111.85 86.975) (end 111.85 86.985) (width 0.25) (layer B.Cu) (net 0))
 (segment (start 111.85 86.985) (end 110.19 88.645) (width 0.25) (layer B.Cu) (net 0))
 (segment (start 110.19 88.645) (end 103.43 88.645) (width 0.25) (layer B.Cu) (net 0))
 (via (at 103.43 88.645) (size 0.6) (drill 0.4) (layers F.Cu B.Cu) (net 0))
 (segment (start 103.43 88.645) (end 103.01 88.225) (width 0.25) (layer F.Cu) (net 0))
 (segment (start 103.01 88.225) (end 100.45 88.225) (width 0.25) (layer F.Cu) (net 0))
 (segment (start 107.049 99.272) (end 107.049 96.876) (width 0.25) (layer F.Cu) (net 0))
 (segment (start 107.049 96.876) (end 107.05 96.875) (width 0.25) (layer F.Cu) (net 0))
 (segment (start 102.87 99.78) (end 105.041 99.78) (width 0.25) (layer F.Cu) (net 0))
 (segment (start 105.041 99.78) (end 105.549 99.272) (width 0.25) (layer F.Cu) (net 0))
 (segment (start 98.9 92.975) (end 98.9 94.352) (width 0.25) (layer F.Cu) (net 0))
 (segment (start 98.9 94.352) (end 97.282 95.97) (width 0.25) (layer F.Cu) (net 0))
 (segment (start 91.75 88.225) (end 93.724 88.225) (width 0.25) (layer F.Cu) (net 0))
 (segment (start 97.282 98.002) (end 97.282 99.78) (width 0.25) (layer F.Cu) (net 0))
 (via (at 97.282 98.002) (size 0.6) (drill 0.4) (layers F.Cu B.Cu) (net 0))
 (segment (start 97.282 91.779) (end 97.282 98.002) (width 0.25) (layer B.Cu) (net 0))
 (segment (start 93.726 88.223) (end 97.282 91.779) (width 0.25) (layer B.Cu) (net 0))
 (via (at 93.726 88.223) (size 0.6) (drill 0.4) (layers F.Cu B.Cu) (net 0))
 (segment (start 93.724 88.225) (end 93.726 88.223) (width 0.25) (layer F.Cu) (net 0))
 (segment (start 90.65 81.375) (end 90.65 84.725) (width 0.25) (layer F.Cu) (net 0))
 (segment (start 90.65 84.725) (end 91.75 85.825) (width 0.25) (layer F.Cu) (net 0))
 (segment (start 94.1 84.275) (end 94.1 82.285) (width 0.25) (layer F.Cu) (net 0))
 (segment (start 94.1 82.285) (end 93.19 81.375) (width 0.25) (layer F.Cu) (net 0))
 (segment (start 108.75 95.175) (end 108.75 95.575) (width 0.25) (layer F.Cu) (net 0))
 (segment (start 100.45 91.425) (end 105.9 96.875) (width 0.25) (layer F.Cu) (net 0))
 (segment (start 107.05 96.875) (end 108.75 95.175) (width 0.25) (layer F.Cu) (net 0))
 (segment (start 105.9 96.875) (end 107.05 96.875) (width 0.25) (layer F.Cu) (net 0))
 (segment (start 107.8 92.375) (end 107.8 90.9) (width 0.25) (layer F.Cu) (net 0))
 (segment (start 107.8 90.9) (end 107.8 85.325) (width 0.25) (layer F.Cu) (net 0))
 (segment (start 107.8 85.325) (end 109.35 84.975) (width 0.25) (layer F.Cu) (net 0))
 (segment (start 108.75 92.375) (end 108.75 93.725) (width 0.25) (layer F.Cu) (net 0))
 (segment (start 106.85 93.675) (end 106.85 92.375) (width 0.25) (layer F.Cu) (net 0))
 (segment (start 108.7 93.675) (end 106.85 93.675) (width 0.25) (layer F.Cu) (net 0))
 (segment (start 108.75 93.725) (end 108.7 93.675) (width 0.25) (layer F.Cu) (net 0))
 (segment (start 108.75 92.375) (end 108.75 89.85) (width 0.25) (layer F.Cu) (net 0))
 (segment (start 108.75 89.85) (end 108.75 87.575) (width 0.25) (layer F.Cu) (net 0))
 (segment (start 108.75 87.575) (end 109.35 86.975) (width 0.25) (layer F.Cu) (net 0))
 (segment (start 92 83.075) (end 92 84.525) (width 0.25) (layer B.Cu) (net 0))
 (segment (start 95.86387 81.748866) (end 94.742 83.016) (width 0.25) (layer B.Cu) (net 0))
 (segment (start 94.742 83.016) (end 92 83.075) (width 0.25) (layer B.Cu) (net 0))
 (segment (start 95.885 81.725) (end 95.86387 81.748866) (width 0.25) (layer B.Cu) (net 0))
 (segment (start 98.9 92.975) (end 100.45 92.975) (width 0.25) (layer F.Cu) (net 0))
 (segment (start 92.25 84.275) (end 93.3 84.275) (width 0.25) (layer F.Cu) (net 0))
 (segment (start 92 84.525) (end 92.25 84.275) (width 0.25) (layer F.Cu) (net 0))
 (via (at 92 84.525) (size 0.6) (drill 0.4) (layers F.Cu B.Cu) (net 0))
 (segment (start 100.45 92.975) (end 97.25 89.775) (width 0.25) (layer B.Cu) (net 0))
 (segment (start 97.25 89.775) (end 92 84.525) (width 0.25) (layer B.Cu) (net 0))
 (via (at 100.45 92.975) (size 0.6) (drill 0.4) (layers F.Cu B.Cu) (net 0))
 (segment (start 91.75 89.025) (end 96.2 89.025) (width 0.25) (layer F.Cu) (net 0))
 (segment (start 96.2 89.025) (end 98.6 91.425) (width 0.25) (layer F.Cu) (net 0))
 (segment (start 98.6 91.425) (end 100.45 91.425) (width 0.25) (layer F.Cu) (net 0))
 (segment (start 93 85.825) (end 96.2 89.025) (width 0.25) (layer F.Cu) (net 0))
 (segment (start 91.75 85.825) (end 93 85.825) (width 0.25) (layer F.Cu) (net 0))
 (segment (start 96.5 92.975) (end 96.5 94.375) (width 0.25) (layer F.Cu) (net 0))
 (segment (start 91.984 98.891) (end 85.598 98.891) (width 0.25) (layer F.Cu) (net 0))
 (segment (start 96.5 94.375) (end 91.984 98.891) (width 0.25) (layer F.Cu) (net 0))
 (segment (start 95.7 92.975) (end 95.7 94.125) (width 0.25) (layer F.Cu) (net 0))
 (segment (start 93.474 96.351) (end 85.598 96.351) (width 0.25) (layer F.Cu) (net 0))
 (segment (start 95.7 94.125) (end 93.474 96.351) (width 0.25) (layer F.Cu) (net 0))
 (segment (start 94.9 92.975) (end 94.9 93.975) (width 0.25) (layer F.Cu) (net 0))
 (segment (start 86.962 95.175) (end 85.598 93.811) (width 0.25) (layer F.Cu) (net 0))
 (segment (start 93.7 95.175) (end 86.962 95.175) (width 0.25) (layer F.Cu) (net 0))
 (segment (start 94.9 93.975) (end 93.7 95.175) (width 0.25) (layer F.Cu) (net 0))
 (segment (start 94.1 92.975) (end 94.1 94.125) (width 0.25) (layer F.Cu) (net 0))
 (segment (start 88.902 94.575) (end 85.598 91.271) (width 0.25) (layer F.Cu) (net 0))
 (segment (start 93.65 94.575) (end 88.902 94.575) (width 0.25) (layer F.Cu) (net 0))
 (segment (start 94.1 94.125) (end 93.65 94.575) (width 0.25) (layer F.Cu) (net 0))
 (segment (start 93.3 92.975) (end 89.842 92.975) (width 0.25) (layer F.Cu) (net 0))
 (segment (start 89.842 92.975) (end 85.598 88.731) (width 0.25) (layer F.Cu) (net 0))
 (segment (start 91.75 91.425) (end 90.25 91.425) (width 0.25) (layer F.Cu) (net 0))
 (segment (start 87.95 88.543) (end 85.598 86.191) (width 0.25) (layer F.Cu) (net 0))
 (segment (start 87.95 89.125) (end 87.95 88.543) (width 0.25) (layer F.Cu) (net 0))
 (segment (start 90.25 91.425) (end 87.95 89.125) (width 0.25) (layer F.Cu) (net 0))
 (segment (start 91.75 90.625) (end 90.15 90.625) (width 0.25) (layer F.Cu) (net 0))
 (segment (start 88.45 86.503) (end 85.598 83.651) (width 0.25) (layer F.Cu) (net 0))
 (segment (start 88.45 88.925) (end 88.45 86.503) (width 0.25) (layer F.Cu) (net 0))
 (segment (start 90.15 90.625) (end 88.45 88.925) (width 0.25) (layer F.Cu) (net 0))
 (segment (start 91.75 89.825) (end 90.15 89.825) (width 0.25) (layer F.Cu) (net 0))
 (segment (start 89 84.513) (end 85.598 81.111) (width 0.25) (layer F.Cu) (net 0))
 (segment (start 89 88.675) (end 89 84.513) (width 0.25) (layer F.Cu) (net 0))
 (segment (start 90.15 89.825) (end 89 88.675) (width 0.25) (layer F.Cu) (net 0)))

